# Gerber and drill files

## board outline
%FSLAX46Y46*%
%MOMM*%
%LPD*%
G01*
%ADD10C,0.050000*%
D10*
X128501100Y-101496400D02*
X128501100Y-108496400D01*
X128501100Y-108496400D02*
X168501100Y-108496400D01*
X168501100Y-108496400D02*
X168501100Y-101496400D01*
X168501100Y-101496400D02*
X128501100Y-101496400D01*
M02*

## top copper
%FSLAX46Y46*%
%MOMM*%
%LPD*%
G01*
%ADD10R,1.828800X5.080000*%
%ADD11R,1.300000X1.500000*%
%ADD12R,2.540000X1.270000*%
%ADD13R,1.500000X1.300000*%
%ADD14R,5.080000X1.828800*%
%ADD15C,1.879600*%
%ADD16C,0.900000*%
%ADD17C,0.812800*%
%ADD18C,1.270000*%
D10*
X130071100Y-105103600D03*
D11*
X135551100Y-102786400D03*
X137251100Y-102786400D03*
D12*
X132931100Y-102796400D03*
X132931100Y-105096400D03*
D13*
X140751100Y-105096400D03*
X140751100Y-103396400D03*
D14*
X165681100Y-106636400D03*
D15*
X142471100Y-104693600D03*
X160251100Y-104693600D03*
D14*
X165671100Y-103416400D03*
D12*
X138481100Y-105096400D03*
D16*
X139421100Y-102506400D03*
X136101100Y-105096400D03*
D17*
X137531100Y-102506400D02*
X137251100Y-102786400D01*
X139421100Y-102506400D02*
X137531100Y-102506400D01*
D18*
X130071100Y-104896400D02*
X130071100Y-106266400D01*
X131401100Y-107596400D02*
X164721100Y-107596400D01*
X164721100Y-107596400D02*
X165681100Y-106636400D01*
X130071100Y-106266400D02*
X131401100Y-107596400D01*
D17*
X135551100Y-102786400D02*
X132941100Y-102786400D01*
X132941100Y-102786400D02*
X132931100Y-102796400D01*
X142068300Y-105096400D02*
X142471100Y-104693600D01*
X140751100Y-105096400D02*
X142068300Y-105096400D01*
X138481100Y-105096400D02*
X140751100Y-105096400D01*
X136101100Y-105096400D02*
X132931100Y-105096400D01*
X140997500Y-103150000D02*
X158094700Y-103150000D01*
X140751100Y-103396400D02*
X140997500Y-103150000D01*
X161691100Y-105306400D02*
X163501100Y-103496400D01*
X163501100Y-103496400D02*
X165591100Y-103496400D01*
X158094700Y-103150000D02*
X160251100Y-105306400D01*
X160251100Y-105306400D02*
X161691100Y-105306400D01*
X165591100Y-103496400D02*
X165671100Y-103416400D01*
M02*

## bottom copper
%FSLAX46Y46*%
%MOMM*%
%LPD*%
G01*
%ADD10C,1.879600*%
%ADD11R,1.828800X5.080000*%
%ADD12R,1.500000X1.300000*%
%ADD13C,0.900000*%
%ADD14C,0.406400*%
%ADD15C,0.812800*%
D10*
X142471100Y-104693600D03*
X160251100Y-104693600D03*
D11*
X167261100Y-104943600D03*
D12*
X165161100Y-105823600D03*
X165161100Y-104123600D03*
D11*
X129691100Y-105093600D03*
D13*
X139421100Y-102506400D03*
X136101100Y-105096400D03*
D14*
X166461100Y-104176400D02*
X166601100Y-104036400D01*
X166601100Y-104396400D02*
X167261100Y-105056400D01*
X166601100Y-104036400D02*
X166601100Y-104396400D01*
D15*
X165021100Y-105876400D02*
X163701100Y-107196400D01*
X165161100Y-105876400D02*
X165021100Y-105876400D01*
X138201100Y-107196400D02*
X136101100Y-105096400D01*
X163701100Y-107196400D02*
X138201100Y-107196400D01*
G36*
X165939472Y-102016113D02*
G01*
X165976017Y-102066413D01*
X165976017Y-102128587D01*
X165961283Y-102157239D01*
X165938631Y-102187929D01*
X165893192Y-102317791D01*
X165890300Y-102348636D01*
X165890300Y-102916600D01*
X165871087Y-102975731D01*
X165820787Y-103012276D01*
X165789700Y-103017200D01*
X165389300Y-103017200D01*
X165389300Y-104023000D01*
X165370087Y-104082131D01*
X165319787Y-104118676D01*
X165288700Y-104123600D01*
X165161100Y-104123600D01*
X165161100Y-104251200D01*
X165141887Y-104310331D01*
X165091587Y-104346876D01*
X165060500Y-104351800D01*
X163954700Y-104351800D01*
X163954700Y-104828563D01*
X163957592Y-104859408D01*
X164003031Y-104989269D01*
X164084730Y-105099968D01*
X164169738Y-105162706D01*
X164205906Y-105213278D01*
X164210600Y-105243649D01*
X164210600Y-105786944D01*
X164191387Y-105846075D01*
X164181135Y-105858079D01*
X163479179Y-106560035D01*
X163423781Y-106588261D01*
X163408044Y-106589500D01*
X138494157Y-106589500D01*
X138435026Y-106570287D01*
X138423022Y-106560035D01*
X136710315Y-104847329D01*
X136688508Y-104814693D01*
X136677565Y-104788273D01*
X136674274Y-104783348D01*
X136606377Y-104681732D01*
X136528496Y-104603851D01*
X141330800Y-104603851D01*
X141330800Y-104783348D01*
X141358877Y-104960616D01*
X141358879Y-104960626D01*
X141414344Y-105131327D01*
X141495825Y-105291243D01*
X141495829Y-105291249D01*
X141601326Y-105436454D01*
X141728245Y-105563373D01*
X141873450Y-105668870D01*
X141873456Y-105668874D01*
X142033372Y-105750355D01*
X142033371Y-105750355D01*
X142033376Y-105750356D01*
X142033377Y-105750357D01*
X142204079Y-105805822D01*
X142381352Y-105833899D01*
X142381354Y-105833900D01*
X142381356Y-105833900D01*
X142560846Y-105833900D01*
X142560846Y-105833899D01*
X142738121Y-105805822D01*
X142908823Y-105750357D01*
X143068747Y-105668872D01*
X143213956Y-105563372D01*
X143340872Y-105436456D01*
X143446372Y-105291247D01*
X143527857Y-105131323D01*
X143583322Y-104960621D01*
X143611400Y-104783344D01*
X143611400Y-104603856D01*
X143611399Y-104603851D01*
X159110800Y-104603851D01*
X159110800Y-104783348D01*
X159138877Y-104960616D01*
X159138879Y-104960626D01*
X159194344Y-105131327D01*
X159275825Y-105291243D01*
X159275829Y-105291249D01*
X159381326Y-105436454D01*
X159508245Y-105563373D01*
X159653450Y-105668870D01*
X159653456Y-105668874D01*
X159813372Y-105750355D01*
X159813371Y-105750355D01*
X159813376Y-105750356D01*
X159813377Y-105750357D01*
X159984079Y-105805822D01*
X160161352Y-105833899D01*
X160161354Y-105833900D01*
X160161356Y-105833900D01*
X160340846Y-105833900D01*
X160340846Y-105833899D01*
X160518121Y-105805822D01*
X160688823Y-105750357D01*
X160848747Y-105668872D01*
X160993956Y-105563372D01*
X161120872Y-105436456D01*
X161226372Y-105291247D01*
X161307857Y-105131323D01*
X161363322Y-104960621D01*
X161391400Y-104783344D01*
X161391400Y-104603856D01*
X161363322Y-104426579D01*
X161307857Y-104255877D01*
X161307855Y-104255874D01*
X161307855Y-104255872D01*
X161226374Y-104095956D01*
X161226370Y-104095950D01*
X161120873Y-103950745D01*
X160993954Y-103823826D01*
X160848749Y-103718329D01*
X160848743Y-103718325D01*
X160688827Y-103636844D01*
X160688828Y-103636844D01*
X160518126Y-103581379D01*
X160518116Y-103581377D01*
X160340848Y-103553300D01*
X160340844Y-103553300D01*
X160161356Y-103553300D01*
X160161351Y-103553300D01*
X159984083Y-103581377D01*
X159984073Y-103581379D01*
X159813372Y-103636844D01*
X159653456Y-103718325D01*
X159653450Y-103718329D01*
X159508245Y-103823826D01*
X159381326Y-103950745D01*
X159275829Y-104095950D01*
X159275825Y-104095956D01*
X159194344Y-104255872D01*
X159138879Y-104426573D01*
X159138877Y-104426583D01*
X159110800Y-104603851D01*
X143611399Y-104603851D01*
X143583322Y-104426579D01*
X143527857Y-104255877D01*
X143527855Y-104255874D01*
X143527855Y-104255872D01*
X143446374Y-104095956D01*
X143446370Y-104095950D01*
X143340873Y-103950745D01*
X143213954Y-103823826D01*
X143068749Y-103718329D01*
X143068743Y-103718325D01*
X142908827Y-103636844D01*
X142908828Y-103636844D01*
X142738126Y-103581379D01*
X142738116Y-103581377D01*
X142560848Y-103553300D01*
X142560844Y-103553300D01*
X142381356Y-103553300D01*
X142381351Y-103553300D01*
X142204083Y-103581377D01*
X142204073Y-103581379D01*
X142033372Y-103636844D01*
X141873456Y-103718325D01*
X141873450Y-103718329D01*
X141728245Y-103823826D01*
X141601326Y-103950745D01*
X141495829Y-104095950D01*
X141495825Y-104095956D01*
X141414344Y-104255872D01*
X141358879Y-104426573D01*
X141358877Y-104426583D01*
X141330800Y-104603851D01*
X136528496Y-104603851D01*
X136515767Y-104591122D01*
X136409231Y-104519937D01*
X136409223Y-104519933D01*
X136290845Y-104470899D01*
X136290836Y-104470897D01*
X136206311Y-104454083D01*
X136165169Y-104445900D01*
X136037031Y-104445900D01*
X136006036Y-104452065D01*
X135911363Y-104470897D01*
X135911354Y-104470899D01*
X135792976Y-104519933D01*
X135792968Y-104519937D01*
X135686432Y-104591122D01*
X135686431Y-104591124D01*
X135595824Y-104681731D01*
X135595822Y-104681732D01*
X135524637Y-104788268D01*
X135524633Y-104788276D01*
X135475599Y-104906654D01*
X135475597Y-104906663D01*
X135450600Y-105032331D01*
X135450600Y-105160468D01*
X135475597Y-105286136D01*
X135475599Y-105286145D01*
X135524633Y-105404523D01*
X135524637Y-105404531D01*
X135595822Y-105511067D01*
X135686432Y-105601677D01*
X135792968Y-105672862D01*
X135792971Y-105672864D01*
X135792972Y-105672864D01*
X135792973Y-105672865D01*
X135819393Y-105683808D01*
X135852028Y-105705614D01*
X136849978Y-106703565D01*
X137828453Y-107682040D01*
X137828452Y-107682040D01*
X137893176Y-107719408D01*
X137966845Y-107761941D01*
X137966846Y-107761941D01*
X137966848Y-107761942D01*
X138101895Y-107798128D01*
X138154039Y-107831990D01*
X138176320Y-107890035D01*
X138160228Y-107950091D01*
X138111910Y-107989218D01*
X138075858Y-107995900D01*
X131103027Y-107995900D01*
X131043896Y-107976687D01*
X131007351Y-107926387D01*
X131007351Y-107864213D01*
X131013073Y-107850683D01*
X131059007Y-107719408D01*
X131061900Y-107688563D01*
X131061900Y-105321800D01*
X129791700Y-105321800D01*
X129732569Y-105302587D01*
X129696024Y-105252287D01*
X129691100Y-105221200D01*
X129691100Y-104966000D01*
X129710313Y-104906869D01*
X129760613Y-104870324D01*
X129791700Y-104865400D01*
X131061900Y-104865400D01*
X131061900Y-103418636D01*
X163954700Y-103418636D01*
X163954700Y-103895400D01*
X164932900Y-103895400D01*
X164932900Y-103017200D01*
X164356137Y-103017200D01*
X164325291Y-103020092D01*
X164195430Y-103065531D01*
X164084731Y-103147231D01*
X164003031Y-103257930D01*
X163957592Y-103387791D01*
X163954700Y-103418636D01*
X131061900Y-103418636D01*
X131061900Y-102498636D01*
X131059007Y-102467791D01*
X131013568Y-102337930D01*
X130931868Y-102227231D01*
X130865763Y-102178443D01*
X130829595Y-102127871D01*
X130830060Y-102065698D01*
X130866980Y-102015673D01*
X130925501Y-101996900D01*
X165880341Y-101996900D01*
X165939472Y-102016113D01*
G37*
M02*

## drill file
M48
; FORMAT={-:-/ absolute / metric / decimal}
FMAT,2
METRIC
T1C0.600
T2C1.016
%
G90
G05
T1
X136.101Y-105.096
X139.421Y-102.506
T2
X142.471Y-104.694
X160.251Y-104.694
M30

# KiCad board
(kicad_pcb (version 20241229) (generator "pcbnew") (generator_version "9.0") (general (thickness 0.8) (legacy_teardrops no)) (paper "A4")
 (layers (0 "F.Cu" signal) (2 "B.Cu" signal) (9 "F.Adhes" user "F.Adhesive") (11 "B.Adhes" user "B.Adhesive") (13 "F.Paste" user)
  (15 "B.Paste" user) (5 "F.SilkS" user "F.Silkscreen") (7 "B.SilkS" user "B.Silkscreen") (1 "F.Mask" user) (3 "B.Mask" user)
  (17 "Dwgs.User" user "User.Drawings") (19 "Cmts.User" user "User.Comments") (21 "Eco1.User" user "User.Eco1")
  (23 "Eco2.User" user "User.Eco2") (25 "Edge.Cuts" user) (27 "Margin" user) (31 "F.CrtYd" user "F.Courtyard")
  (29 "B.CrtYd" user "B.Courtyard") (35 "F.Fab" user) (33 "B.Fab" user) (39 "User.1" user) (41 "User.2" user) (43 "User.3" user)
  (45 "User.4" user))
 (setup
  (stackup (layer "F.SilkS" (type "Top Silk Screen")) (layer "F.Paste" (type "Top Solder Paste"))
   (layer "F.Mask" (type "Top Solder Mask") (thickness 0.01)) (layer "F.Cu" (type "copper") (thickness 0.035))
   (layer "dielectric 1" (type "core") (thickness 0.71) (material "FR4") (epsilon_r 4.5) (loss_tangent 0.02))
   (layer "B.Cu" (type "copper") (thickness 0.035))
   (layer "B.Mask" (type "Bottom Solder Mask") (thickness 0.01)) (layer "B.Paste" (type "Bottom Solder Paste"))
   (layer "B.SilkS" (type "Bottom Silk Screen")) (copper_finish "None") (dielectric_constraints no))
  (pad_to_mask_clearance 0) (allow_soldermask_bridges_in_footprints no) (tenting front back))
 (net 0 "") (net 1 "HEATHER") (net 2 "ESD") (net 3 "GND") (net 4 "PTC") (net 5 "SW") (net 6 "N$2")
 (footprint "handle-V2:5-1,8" (layer "F.Cu") (at 130.0711 105.1036 180)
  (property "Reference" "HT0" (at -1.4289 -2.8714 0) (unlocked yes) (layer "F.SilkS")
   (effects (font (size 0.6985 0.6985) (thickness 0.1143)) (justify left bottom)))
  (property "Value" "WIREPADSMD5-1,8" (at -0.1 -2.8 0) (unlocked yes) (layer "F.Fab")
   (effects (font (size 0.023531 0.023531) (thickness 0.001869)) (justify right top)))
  (pad "1" smd rect (at 0 0 180) (size 1.8288 5.08) (layers "F.Cu" "F.Mask" "F.Paste") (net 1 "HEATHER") (solder_mask_margin 0)
   (solder_paste_margin 0) (thermal_bridge_angle 0)))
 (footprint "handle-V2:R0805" (layer "F.Cu") (at 136.4011 102.7864)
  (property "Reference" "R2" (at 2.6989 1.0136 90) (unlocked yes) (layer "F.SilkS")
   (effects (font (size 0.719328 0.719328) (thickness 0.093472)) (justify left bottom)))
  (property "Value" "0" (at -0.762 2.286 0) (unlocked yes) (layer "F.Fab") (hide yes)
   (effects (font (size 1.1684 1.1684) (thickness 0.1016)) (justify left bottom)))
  (pad "1" smd rect (at -0.85 0) (size 1.3 1.5) (layers "F.Cu" "F.Mask" "F.Paste") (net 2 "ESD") (solder_mask_margin 0)
   (solder_paste_margin 0) (thermal_bridge_angle 0))
  (pad "2" smd rect (at 0.85 0) (size 1.3 1.5) (layers "F.Cu" "F.Mask" "F.Paste") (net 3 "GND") (solder_mask_margin 0)
   (solder_paste_margin 0) (thermal_bridge_angle 0)))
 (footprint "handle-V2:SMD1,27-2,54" (layer "F.Cu") (at 132.9311 102.7964 -90)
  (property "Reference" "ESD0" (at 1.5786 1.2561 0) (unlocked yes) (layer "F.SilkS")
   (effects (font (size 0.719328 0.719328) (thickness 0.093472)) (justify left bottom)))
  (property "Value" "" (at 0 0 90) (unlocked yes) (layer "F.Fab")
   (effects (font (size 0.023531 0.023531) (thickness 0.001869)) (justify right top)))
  (pad "1" smd rect (at 0 0 270) (size 1.27 2.54) (layers "F.Cu" "F.Mask" "F.Paste") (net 2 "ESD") (solder_mask_margin 0)
   (solder_paste_margin 0) (thermal_bridge_angle 0)))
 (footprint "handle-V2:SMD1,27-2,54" (layer "F.Cu") (at 132.9311 105.0964 -90)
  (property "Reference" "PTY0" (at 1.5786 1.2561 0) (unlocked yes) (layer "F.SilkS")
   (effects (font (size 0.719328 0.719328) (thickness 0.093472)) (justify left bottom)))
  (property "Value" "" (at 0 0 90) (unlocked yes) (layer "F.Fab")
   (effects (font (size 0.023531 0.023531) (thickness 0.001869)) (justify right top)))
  (pad "1" smd rect (at 0 0 270) (size 1.27 2.54) (layers "F.Cu" "F.Mask" "F.Paste") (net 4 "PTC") (solder_mask_margin 0)
   (solder_paste_margin 0) (thermal_bridge_angle 0)))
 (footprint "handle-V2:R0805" (layer "F.Cu") (at 140.7511 104.2464 90)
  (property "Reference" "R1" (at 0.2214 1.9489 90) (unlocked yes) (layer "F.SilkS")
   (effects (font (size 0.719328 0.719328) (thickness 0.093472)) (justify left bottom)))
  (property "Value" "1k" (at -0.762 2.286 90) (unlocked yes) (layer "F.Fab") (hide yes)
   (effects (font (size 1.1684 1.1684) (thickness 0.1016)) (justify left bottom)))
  (pad "1" smd rect (at -0.85 0 90) (size 1.3 1.5) (layers "F.Cu" "F.Mask" "F.Paste") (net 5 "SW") (solder_mask_margin 0)
   (solder_paste_margin 0) (thermal_bridge_angle 0))
  (pad "2" smd rect (at 0.85 0 90) (size 1.3 1.5) (layers "F.Cu" "F.Mask" "F.Paste") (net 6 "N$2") (solder_mask_margin 0)
   (solder_paste_margin 0) (thermal_bridge_angle 0)))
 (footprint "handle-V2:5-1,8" (layer "F.Cu") (at 165.6811 106.6364 90)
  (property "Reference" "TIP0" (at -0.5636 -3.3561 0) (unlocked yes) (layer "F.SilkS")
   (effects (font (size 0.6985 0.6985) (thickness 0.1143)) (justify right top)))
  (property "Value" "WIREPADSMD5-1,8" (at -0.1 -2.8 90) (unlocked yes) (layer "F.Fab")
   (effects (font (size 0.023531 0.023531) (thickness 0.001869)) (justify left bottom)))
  (pad "1" smd rect (at 0 0 90) (size 1.8288 5.08) (layers "F.Cu" "F.Mask" "F.Paste") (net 1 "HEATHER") (solder_mask_margin 0)
   (solder_paste_margin 0) (thermal_bridge_angle 0)))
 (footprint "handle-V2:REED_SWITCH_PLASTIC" (layer "F.Cu") (at 151.3611 104.6936)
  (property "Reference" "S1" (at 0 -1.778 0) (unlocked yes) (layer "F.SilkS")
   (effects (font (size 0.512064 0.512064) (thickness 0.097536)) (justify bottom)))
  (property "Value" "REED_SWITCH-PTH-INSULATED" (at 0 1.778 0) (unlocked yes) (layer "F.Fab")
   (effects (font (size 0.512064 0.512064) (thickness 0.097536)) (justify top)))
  (pad "P$1" thru_hole circle (at -8.89 0) (size 1.8796 1.8796) (drill 1.016) (layers "*.Cu" "*.Mask") (remove_unused_layers no)
   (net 5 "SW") (solder_mask_margin 0) (thermal_bridge_angle 0))
  (pad "P$2" thru_hole circle (at 8.89 0) (size 1.8796 1.8796) (drill 1.016) (layers "*.Cu" "*.Mask") (remove_unused_layers no)
   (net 6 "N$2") (solder_mask_margin 0) (thermal_bridge_angle 0)))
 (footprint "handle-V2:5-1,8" (layer "F.Cu") (at 165.6711 103.4164 90)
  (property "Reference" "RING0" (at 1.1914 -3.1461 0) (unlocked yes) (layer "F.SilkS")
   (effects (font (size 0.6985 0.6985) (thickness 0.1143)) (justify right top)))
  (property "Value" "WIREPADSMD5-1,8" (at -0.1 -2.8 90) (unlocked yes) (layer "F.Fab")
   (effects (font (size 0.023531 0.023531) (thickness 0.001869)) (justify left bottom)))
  (pad "1" smd rect (at 0 0 90) (size 1.8288 5.08) (layers "F.Cu" "F.Mask" "F.Paste") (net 6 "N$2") (solder_mask_margin 0)
   (solder_paste_margin 0) (thermal_bridge_angle 0)))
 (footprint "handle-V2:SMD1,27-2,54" (layer "F.Cu") (at 138.4811 105.0964 -90)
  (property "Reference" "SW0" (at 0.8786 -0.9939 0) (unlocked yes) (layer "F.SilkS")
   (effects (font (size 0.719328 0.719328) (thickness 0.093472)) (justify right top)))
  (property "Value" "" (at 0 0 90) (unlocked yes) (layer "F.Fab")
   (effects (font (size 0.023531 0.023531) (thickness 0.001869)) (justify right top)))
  (pad "1" smd rect (at 0 0 270) (size 1.27 2.54) (layers "F.Cu" "F.Mask" "F.Paste") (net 5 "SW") (solder_mask_margin 0)
   (solder_paste_margin 0) (thermal_bridge_angle 0)))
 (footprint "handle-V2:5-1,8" (layer "B.Cu") (at 167.2611 104.9436)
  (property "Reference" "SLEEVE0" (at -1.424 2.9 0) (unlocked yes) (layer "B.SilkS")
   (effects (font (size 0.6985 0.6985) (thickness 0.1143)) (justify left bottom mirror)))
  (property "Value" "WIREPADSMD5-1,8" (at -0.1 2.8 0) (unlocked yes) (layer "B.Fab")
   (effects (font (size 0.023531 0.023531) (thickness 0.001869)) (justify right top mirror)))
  (pad "1" smd rect (at 0 0) (size 1.8288 5.08) (layers "B.Cu" "B.Mask" "B.Paste") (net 3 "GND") (solder_mask_margin 0)
   (solder_paste_margin 0) (thermal_bridge_angle 0)))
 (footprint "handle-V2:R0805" (layer "B.Cu") (at 165.1611 104.9736 90)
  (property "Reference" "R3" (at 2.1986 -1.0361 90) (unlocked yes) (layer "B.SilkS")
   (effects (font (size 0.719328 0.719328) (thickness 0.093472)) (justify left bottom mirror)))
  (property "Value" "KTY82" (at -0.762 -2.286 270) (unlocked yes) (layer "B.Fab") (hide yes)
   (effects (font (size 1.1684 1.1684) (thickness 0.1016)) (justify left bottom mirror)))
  (pad "1" smd rect (at -0.85 0 90) (size 1.3 1.5) (layers "B.Cu" "B.Mask" "B.Paste") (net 4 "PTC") (solder_mask_margin 0)
   (solder_paste_margin 0) (thermal_bridge_angle 0))
  (pad "2" smd rect (at 0.85 0 90) (size 1.3 1.5) (layers "B.Cu" "B.Mask" "B.Paste") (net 3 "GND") (solder_mask_margin 0)
   (solder_paste_margin 0) (thermal_bridge_angle 0)))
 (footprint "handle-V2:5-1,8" (layer "B.Cu") (at 129.6911 105.0936)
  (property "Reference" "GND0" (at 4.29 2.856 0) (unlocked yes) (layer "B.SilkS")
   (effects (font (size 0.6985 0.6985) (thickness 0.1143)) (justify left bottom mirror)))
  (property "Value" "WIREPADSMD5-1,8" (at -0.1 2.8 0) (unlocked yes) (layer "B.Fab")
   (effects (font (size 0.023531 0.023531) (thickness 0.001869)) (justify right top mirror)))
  (pad "1" smd rect (at 0 0) (size 1.8288 5.08) (layers "B.Cu" "B.Mask" "B.Paste") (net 3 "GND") (solder_mask_margin 0)
   (solder_paste_margin 0) (thermal_bridge_angle 0)))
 (gr_line (start 128.5011 101.4964) (end 128.5011 108.4964) (stroke (width 0.05) (type solid)) (layer "Edge.Cuts"))
 (gr_line (start 128.5011 108.4964) (end 168.5011 108.4964) (stroke (width 0.05) (type solid)) (layer "Edge.Cuts"))
 (gr_line (start 168.5011 108.4964) (end 168.5011 101.4964) (stroke (width 0.05) (type solid)) (layer "Edge.Cuts"))
 (gr_line (start 168.5011 101.4964) (end 128.5011 101.4964) (stroke (width 0.05) (type solid)) (layer "Edge.Cuts"))
 (segment (start 137.5311 102.5064) (end 137.2511 102.7864) (width 0.8128) (layer "F.Cu") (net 3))
 (segment (start 139.4211 102.5064) (end 137.5311 102.5064) (width 0.8128) (layer "F.Cu") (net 3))
 (via (at 139.4211 102.5064) (size 0.9) (drill 0.6) (layers "F.Cu" "B.Cu") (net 3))
 (segment (start 166.4611 104.1764) (end 166.6011 104.0364) (width 0.4064) (layer "B.Cu") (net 3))
 (segment (start 166.6011 104.3964) (end 167.2611 105.0564) (width 0.4064) (layer "B.Cu") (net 3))
 (segment (start 166.6011 104.0364) (end 166.6011 104.3964) (width 0.4064) (layer "B.Cu") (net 3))
 (segment (start 130.0711 104.8964) (end 130.0711 106.2664) (width 1.27) (layer "F.Cu") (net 1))
 (segment (start 131.4011 107.5964) (end 164.7211 107.5964) (width 1.27) (layer "F.Cu") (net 1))
 (segment (start 164.7211 107.5964) (end 165.6811 106.6364) (width 1.27) (layer "F.Cu") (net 1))
 (segment (start 130.0711 106.2664) (end 131.4011 107.5964) (width 1.27) (layer "F.Cu") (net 1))
 (segment (start 135.5511 102.7864) (end 132.9411 102.7864) (width 0.8128) (layer "F.Cu") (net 2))
 (segment (start 132.9411 102.7864) (end 132.9311 102.7964) (width 0.8128) (layer "F.Cu") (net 2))
 (segment (start 142.0683 105.0964) (end 142.4711 104.6936) (width 0.8128) (layer "F.Cu") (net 5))
 (segment (start 140.7511 105.0964) (end 142.0683 105.0964) (width 0.8128) (layer "F.Cu") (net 5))
 (segment (start 138.4811 105.0964) (end 140.7511 105.0964) (width 0.8128) (layer "F.Cu") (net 5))
 (segment (start 136.1011 105.0964) (end 132.9311 105.0964) (width 0.8128) (layer "F.Cu") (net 4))
 (via (at 136.1011 105.0964) (size 0.9) (drill 0.6) (layers "F.Cu" "B.Cu") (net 4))
 (segment (start 165.0211 105.8764) (end 163.7011 107.1964) (width 0.8128) (layer "B.Cu") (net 4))
 (segment (start 165.1611 105.8764) (end 165.0211 105.8764) (width 0.8128) (layer "B.Cu") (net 4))
 (segment (start 138.2011 107.1964) (end 136.1011 105.0964) (width 0.8128) (layer "B.Cu") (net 4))
 (segment (start 163.7011 107.1964) (end 138.2011 107.1964) (width 0.8128) (layer "B.Cu") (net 4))
 (segment (start 140.9975 103.15) (end 158.0947 103.15) (width 0.8128) (layer "F.Cu") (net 6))
 (segment (start 140.7511 103.3964) (end 140.9975 103.15) (width 0.8128) (layer "F.Cu") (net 6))
 (segment (start 161.6911 105.3064) (end 163.5011 103.4964) (width 0.8128) (layer "F.Cu") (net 6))
 (segment (start 163.5011 103.4964) (end 165.5911 103.4964) (width 0.8128) (layer "F.Cu") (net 6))
 (segment (start 158.0947 103.15) (end 160.2511 105.3064) (width 0.8128) (layer "F.Cu") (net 6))
 (segment (start 160.2511 105.3064) (end 161.6911 105.3064) (width 0.8128) (layer "F.Cu") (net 6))
 (segment (start 165.5911 103.4964) (end 165.6711 103.4164) (width 0.8128) (layer "F.Cu") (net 6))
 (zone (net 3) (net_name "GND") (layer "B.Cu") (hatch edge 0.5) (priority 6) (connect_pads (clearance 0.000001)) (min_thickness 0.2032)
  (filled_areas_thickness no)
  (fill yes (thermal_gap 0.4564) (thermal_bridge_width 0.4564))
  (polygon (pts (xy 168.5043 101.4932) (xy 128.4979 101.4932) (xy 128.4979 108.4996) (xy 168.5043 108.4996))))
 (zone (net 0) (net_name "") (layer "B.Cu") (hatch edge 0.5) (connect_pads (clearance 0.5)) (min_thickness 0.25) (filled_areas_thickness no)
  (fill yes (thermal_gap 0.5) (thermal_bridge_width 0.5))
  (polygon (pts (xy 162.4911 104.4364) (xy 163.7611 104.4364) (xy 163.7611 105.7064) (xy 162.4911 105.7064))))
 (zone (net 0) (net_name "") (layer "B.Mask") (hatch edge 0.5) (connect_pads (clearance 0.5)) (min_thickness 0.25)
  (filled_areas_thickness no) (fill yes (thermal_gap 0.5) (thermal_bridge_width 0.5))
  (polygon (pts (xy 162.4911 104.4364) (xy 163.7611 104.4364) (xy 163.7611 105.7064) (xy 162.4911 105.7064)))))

